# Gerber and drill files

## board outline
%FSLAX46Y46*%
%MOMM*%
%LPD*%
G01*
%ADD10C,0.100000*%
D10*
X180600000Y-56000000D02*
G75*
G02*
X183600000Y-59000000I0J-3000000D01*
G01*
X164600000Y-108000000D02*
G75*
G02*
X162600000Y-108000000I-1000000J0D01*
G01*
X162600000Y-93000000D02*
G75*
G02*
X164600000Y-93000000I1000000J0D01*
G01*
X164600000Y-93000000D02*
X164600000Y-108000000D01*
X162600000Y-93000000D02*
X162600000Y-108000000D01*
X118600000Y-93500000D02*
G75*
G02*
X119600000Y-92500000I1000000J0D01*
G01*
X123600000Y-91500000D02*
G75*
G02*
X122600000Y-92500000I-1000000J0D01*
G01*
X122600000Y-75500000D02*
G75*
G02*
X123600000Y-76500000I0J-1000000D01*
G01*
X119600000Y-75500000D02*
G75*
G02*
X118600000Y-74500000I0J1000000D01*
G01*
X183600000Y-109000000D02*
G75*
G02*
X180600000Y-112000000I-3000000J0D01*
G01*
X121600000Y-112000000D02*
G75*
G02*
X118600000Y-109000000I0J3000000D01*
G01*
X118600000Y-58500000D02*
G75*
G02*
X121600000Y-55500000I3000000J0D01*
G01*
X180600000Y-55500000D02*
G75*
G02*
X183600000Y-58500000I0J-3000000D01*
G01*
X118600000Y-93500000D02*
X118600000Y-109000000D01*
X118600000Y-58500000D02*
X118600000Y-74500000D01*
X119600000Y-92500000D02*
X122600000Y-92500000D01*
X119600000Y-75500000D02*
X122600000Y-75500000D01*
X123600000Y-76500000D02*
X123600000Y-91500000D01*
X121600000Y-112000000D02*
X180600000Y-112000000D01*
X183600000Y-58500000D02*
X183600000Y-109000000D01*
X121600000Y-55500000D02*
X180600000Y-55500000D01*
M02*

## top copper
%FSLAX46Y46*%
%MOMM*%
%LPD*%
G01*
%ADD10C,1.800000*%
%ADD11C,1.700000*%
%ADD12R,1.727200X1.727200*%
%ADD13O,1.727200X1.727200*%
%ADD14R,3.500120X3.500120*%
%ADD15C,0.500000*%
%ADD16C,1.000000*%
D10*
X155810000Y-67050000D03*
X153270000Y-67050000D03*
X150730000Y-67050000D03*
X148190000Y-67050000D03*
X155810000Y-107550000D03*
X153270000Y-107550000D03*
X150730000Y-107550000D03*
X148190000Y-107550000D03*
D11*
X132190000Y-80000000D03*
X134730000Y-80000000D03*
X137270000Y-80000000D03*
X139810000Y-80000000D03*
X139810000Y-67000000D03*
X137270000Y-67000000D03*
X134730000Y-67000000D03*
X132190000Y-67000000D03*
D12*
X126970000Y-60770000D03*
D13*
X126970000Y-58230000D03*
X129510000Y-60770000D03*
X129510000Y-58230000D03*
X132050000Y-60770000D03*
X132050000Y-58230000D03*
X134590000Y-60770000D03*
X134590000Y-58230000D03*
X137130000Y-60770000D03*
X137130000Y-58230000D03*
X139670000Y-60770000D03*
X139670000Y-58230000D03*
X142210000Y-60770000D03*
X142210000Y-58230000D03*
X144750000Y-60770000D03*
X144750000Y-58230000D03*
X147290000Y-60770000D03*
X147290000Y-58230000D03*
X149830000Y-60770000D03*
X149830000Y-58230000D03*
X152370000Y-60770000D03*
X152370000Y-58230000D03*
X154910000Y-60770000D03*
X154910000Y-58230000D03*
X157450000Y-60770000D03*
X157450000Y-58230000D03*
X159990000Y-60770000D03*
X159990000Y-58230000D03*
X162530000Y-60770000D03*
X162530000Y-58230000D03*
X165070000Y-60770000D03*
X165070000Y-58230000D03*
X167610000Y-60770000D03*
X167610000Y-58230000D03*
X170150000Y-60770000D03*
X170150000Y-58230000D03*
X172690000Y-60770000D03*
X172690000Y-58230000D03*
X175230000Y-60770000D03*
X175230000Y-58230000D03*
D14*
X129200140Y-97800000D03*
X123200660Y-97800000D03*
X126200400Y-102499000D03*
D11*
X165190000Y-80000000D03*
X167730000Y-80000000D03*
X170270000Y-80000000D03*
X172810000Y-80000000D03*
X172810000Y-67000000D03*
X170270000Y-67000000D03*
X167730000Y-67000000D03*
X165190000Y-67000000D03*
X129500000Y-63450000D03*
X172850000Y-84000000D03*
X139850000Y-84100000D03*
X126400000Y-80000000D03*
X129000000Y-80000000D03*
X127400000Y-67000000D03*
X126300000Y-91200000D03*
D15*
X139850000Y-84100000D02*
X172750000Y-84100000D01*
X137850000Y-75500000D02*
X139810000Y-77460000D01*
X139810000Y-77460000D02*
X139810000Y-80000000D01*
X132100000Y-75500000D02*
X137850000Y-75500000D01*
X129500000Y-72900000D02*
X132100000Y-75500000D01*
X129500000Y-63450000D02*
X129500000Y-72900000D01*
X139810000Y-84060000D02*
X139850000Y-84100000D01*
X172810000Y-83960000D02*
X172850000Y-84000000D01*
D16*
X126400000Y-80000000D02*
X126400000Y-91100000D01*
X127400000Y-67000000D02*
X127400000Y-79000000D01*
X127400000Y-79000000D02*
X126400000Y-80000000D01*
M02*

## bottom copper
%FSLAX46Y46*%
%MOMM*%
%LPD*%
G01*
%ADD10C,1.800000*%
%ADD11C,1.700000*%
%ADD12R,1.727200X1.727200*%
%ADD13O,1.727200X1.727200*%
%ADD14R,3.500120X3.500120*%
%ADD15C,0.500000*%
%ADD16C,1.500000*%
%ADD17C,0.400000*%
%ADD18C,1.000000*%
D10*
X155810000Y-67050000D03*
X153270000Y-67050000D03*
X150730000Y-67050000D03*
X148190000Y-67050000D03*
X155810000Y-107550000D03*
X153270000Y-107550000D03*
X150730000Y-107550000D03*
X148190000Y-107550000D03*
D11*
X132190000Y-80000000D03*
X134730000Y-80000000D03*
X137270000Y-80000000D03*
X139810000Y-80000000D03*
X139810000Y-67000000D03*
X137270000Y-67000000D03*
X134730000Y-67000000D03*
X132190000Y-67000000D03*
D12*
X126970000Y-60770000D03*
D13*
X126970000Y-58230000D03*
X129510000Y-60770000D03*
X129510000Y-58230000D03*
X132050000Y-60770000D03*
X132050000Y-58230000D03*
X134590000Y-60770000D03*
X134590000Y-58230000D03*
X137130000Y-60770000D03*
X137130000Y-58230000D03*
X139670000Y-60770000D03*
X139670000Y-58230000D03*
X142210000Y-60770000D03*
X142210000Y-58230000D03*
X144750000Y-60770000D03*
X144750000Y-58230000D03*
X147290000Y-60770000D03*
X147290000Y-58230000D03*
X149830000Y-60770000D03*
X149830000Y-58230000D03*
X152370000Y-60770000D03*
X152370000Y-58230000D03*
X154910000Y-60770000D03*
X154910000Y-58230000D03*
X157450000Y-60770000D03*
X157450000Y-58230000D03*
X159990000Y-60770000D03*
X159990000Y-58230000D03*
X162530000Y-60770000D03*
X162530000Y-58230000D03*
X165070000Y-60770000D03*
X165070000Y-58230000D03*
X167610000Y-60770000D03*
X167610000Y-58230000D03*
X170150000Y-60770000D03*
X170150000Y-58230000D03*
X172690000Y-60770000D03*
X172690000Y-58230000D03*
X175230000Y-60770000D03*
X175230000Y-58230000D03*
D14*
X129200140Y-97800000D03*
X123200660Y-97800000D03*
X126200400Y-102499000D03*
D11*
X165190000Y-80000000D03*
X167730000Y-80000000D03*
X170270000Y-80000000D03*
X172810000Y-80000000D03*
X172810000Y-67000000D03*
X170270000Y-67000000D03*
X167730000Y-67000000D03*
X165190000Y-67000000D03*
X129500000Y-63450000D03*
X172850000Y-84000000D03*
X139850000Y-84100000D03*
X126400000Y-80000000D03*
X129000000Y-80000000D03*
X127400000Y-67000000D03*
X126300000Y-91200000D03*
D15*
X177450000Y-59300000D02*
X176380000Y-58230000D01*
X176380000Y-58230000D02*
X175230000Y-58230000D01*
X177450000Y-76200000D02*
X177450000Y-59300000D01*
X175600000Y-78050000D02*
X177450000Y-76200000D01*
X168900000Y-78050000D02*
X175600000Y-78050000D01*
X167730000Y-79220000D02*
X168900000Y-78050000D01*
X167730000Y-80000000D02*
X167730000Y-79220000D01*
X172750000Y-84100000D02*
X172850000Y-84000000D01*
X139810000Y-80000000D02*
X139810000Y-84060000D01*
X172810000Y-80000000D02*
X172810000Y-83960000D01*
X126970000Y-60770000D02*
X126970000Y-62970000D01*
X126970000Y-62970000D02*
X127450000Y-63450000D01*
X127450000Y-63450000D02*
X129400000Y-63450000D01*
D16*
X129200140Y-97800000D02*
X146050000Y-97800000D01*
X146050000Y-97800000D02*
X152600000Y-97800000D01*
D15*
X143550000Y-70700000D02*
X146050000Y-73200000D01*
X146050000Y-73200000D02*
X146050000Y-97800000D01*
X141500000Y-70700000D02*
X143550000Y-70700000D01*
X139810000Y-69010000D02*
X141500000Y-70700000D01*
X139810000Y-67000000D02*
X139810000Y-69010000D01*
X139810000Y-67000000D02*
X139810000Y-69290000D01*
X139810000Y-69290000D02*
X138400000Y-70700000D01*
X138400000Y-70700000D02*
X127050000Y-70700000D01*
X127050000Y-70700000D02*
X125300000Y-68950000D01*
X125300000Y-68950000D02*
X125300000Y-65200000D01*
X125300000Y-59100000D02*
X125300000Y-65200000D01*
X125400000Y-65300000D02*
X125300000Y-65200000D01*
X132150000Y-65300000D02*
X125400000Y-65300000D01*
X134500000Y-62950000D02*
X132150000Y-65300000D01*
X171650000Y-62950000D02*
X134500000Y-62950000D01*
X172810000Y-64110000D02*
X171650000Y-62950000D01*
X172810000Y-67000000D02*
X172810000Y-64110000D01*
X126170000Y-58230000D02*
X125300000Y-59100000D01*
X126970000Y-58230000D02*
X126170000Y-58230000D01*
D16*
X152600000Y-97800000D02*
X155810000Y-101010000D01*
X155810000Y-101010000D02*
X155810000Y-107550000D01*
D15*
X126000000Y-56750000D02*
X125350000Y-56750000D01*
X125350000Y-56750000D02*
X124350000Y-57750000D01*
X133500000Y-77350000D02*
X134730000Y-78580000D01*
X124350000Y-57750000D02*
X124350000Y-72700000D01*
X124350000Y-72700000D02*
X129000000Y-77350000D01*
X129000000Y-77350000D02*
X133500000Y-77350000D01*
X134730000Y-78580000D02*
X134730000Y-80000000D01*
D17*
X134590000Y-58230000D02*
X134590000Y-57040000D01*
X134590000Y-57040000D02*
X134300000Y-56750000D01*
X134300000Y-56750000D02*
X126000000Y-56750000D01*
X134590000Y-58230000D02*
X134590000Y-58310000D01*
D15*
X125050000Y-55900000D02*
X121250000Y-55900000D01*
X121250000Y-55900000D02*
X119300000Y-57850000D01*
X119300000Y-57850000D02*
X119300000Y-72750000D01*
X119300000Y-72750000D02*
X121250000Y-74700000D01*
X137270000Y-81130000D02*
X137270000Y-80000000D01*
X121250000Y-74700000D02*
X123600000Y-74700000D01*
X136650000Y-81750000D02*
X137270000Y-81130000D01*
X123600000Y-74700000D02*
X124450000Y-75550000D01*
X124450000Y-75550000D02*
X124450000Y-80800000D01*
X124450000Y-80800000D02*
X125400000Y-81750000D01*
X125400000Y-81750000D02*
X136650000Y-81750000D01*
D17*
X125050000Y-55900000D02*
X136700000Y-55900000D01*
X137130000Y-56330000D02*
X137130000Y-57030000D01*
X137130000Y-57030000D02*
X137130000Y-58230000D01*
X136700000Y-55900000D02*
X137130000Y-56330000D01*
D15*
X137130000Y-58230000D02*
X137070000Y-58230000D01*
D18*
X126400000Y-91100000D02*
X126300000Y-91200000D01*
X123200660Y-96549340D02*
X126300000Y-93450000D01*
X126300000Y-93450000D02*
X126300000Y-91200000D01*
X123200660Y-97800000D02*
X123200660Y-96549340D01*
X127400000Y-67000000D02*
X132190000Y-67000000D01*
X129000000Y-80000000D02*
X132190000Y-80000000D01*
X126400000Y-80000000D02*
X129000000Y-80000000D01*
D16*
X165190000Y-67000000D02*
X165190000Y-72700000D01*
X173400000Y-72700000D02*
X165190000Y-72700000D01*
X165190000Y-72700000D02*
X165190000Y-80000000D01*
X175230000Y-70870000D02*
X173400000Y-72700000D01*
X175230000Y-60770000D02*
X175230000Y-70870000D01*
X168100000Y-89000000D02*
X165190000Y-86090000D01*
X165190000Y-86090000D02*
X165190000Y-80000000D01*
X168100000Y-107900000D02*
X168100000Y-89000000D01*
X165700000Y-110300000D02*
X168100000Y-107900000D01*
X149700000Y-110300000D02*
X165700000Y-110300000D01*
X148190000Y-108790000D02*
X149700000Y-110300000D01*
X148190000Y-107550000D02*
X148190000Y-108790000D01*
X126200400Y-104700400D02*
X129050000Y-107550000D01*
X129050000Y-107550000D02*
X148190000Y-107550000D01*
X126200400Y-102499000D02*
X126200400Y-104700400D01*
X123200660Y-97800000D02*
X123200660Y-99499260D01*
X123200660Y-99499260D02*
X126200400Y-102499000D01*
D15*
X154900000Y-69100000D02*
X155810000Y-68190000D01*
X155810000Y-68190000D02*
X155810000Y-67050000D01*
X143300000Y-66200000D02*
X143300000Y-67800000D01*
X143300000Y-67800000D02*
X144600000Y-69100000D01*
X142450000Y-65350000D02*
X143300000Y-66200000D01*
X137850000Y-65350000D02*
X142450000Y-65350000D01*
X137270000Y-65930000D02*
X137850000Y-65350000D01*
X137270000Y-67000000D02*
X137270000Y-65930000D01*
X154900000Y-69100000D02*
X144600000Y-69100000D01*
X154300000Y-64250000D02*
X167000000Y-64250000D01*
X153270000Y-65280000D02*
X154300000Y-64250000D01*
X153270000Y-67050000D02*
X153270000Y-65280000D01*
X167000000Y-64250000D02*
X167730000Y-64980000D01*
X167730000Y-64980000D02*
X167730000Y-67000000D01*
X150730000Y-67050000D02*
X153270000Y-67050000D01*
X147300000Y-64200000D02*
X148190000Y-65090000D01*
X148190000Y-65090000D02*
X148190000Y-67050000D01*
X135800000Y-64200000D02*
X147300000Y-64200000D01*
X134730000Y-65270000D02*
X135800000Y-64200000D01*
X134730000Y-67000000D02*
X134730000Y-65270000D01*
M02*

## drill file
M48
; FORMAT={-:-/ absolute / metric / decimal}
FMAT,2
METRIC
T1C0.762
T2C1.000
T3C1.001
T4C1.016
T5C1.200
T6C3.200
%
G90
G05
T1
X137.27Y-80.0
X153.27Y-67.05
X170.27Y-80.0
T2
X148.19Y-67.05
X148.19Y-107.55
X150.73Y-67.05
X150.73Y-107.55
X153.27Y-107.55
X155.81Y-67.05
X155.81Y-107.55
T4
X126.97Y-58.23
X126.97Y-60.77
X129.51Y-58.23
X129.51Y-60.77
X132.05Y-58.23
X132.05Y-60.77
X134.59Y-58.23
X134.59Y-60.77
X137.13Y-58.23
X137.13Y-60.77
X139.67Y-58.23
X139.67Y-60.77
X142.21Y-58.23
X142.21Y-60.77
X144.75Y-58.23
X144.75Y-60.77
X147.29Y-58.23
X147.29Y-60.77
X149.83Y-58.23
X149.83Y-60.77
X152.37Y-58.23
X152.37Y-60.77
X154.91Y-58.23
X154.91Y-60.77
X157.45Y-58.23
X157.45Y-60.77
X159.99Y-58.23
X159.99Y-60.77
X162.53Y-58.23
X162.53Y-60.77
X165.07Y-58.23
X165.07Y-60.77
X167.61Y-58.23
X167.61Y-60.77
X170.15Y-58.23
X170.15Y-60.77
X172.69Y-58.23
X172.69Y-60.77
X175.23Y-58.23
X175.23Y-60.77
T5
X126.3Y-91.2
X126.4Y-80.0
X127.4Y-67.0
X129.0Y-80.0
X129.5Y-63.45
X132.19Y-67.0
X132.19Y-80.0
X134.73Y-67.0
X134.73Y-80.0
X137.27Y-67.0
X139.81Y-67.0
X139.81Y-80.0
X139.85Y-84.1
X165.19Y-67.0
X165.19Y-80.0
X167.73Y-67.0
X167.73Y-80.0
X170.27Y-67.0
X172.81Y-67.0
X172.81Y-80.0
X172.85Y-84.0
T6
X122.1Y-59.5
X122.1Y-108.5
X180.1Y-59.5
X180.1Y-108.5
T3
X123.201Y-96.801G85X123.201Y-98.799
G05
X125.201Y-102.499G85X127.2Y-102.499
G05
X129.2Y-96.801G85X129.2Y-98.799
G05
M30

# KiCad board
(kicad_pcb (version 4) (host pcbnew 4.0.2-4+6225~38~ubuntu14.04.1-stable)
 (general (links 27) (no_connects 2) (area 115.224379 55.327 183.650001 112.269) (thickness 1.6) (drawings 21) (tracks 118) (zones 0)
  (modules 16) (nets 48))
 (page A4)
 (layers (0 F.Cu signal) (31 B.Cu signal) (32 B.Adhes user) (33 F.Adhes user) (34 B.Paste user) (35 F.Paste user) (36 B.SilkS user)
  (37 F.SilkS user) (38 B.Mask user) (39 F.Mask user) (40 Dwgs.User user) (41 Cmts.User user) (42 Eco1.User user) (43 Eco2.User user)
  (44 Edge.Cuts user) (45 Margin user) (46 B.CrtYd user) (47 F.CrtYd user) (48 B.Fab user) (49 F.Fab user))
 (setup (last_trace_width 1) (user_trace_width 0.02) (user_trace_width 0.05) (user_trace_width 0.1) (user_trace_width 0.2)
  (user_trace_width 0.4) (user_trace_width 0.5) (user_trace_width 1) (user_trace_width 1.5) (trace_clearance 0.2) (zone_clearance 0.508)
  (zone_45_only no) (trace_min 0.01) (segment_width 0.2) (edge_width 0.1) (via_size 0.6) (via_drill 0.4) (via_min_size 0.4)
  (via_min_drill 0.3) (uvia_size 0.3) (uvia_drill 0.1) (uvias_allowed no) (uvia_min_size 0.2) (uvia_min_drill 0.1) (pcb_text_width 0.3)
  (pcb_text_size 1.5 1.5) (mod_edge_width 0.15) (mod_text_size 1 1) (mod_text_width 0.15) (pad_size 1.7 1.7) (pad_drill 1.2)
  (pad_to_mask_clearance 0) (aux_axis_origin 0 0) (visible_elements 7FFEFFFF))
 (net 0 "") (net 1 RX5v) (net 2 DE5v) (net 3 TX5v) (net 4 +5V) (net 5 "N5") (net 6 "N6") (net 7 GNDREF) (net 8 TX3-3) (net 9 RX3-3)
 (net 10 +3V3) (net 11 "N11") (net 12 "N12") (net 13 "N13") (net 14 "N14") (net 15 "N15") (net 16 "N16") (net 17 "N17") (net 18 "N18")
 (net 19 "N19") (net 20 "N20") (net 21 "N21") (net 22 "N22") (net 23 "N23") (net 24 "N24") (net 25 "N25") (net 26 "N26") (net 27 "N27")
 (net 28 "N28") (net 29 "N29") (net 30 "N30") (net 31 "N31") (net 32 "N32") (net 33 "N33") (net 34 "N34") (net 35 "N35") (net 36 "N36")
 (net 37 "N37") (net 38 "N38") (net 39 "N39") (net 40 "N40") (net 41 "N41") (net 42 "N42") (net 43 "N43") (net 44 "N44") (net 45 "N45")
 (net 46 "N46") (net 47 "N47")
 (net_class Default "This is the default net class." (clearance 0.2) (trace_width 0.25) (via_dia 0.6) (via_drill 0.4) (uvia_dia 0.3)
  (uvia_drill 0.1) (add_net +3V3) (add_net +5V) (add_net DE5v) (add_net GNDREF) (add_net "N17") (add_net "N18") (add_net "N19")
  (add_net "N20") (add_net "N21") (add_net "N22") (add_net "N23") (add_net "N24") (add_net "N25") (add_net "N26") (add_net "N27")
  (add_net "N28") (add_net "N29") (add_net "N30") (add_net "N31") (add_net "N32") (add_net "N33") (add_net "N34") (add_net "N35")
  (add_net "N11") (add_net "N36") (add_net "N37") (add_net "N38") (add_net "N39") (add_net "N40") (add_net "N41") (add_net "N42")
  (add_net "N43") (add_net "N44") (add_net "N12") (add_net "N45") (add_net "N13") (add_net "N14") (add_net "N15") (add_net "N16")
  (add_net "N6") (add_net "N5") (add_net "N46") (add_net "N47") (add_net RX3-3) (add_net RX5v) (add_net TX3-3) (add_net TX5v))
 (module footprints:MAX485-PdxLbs (layer F.Cu) (at 152 87.3 180)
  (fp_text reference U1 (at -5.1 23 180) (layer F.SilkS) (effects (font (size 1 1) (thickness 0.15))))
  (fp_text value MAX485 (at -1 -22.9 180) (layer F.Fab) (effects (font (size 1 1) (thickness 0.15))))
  (pad 1 thru_hole circle (at -3.81 20.25 180) (size 1.8 1.8) (drill 1) (layers *.Cu *.Mask F.SilkS) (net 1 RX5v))
  (pad 2 thru_hole circle (at -1.27 20.25 180) (size 1.8 1.8) (drill 0.762) (layers *.Cu *.Mask F.SilkS) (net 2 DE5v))
  (pad 3 thru_hole circle (at 1.27 20.25 180) (size 1.8 1.8) (drill 1) (layers *.Cu *.Mask F.SilkS) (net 2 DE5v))
  (pad 4 thru_hole circle (at 3.81 20.25 180) (size 1.8 1.8) (drill 1) (layers *.Cu *.Mask F.SilkS) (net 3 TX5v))
  (pad 8 thru_hole circle (at -3.81 -20.25 180) (size 1.8 1.8) (drill 1) (layers *.Cu *.Mask F.SilkS) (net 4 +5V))
  (pad 7 thru_hole circle (at -1.27 -20.25 180) (size 1.8 1.8) (drill 1) (layers *.Cu *.Mask F.SilkS) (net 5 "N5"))
  (pad 6 thru_hole circle (at 1.27 -20.25 180) (size 1.8 1.8) (drill 1) (layers *.Cu *.Mask F.SilkS) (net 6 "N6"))
  (pad 5 thru_hole circle (at 3.81 -20.25 180) (size 1.8 1.8) (drill 1) (layers *.Cu *.Mask F.SilkS) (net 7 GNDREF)))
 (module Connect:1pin (layer F.Cu) (at 180.1 59.5)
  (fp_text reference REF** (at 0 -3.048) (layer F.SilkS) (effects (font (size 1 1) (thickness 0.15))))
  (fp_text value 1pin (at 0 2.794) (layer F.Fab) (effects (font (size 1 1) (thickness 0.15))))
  (pad "" np_thru_hole circle (at 0 0) (size 3.2 3.2) (drill 3.2) (layers *.Cu *.Mask F.SilkS)))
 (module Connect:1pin (layer F.Cu) (at 180.1 108.5)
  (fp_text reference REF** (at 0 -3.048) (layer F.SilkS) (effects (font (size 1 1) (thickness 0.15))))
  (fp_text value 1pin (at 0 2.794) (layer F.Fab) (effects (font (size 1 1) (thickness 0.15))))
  (pad "" np_thru_hole circle (at 0 0) (size 3.2 3.2) (drill 3.2) (layers *.Cu *.Mask F.SilkS)))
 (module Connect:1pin (layer F.Cu) (at 122.1 108.5)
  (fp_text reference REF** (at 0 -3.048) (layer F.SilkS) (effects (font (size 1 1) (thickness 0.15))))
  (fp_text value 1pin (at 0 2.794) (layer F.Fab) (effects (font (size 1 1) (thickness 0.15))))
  (pad "" np_thru_hole circle (at 0 0) (size 3.2 3.2) (drill 3.2) (layers *.Cu *.Mask F.SilkS)))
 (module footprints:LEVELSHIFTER (layer F.Cu) (at 136 73.5 90)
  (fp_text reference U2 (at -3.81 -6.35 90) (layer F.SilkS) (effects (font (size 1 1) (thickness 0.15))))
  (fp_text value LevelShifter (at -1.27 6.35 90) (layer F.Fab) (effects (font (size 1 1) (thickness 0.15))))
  (pad 1 thru_hole circle (at -6.5 -3.81 90) (size 1.7 1.7) (drill 1.2) (layers *.Cu *.Mask F.SilkS) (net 7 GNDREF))
  (pad 2 thru_hole circle (at -6.5 -1.27 90) (size 1.7 1.7) (drill 1.2) (layers *.Cu *.Mask F.SilkS) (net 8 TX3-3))
  (pad 3 thru_hole circle (at -6.5 1.27 90) (size 1.7 1.7) (drill 0.762) (layers *.Cu *.Mask F.SilkS) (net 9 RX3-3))
  (pad 4 thru_hole circle (at -6.5 3.81 90) (size 1.7 1.7) (drill 1.2) (layers *.Cu *.Mask F.SilkS) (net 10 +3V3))
  (pad 5 thru_hole circle (at 6.5 3.81 90) (size 1.7 1.7) (drill 1.2) (layers *.Cu *.Mask F.SilkS) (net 4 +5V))
  (pad 6 thru_hole circle (at 6.5 1.27 90) (size 1.7 1.7) (drill 1.2) (layers *.Cu *.Mask F.SilkS) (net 1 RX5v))
  (pad 7 thru_hole circle (at 6.5 -1.27 90) (size 1.7 1.7) (drill 1.2) (layers *.Cu *.Mask F.SilkS) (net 3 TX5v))
  (pad 8 thru_hole circle (at 6.5 -3.81 90) (size 1.7 1.7) (drill 1.2) (layers *.Cu *.Mask F.SilkS) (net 7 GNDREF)))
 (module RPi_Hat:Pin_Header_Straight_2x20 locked (layer F.Cu) (at 151.1 59.5 90)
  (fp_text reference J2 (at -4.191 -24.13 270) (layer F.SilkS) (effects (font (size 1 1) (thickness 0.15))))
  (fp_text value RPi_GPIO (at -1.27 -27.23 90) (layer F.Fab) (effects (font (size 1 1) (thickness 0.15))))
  (pad 1 thru_hole rect (at -1.27 -24.13 90) (size 1.7272 1.7272) (drill 1.016) (layers *.Cu *.Mask F.SilkS) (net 10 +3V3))
  (pad 2 thru_hole oval (at 1.27 -24.13 90) (size 1.7272 1.7272) (drill 1.016) (layers *.Cu *.Mask F.SilkS) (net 4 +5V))
  (pad 3 thru_hole oval (at -1.27 -21.59 90) (size 1.7272 1.7272) (drill 1.016) (layers *.Cu *.Mask F.SilkS) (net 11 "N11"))
  (pad 4 thru_hole oval (at 1.27 -21.59 90) (size 1.7272 1.7272) (drill 1.016) (layers *.Cu *.Mask F.SilkS) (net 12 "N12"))
  (pad 5 thru_hole oval (at -1.27 -19.05 90) (size 1.7272 1.7272) (drill 1.016) (layers *.Cu *.Mask F.SilkS) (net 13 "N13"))
  (pad 6 thru_hole oval (at 1.27 -19.05 90) (size 1.7272 1.7272) (drill 1.016) (layers *.Cu *.Mask F.SilkS) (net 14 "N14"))
  (pad 7 thru_hole oval (at -1.27 -16.51 90) (size 1.7272 1.7272) (drill 1.016) (layers *.Cu *.Mask F.SilkS) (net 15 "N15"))
  (pad 8 thru_hole oval (at 1.27 -16.51 90) (size 1.7272 1.7272) (drill 1.016) (layers *.Cu *.Mask F.SilkS) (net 8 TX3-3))
  (pad 9 thru_hole oval (at -1.27 -13.97 90) (size 1.7272 1.7272) (drill 1.016) (layers *.Cu *.Mask F.SilkS) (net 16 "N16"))
  (pad 10 thru_hole oval (at 1.27 -13.97 90) (size 1.7272 1.7272) (drill 1.016) (layers *.Cu *.Mask F.SilkS) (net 9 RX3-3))
  (pad 11 thru_hole oval (at -1.27 -11.43 90) (size 1.7272 1.7272) (drill 1.016) (layers *.Cu *.Mask F.SilkS) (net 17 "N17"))
  (pad 12 thru_hole oval (at 1.27 -11.43 90) (size 1.7272 1.7272) (drill 1.016) (layers *.Cu *.Mask F.SilkS) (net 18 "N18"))
  (pad 13 thru_hole oval (at -1.27 -8.89 90) (size 1.7272 1.7272) (drill 1.016) (layers *.Cu *.Mask F.SilkS) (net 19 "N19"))
  (pad 14 thru_hole oval (at 1.27 -8.89 90) (size 1.7272 1.7272) (drill 1.016) (layers *.Cu *.Mask F.SilkS) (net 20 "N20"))
  (pad 15 thru_hole oval (at -1.27 -6.35 90) (size 1.7272 1.7272) (drill 1.016) (layers *.Cu *.Mask F.SilkS) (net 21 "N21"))
  (pad 16 thru_hole oval (at 1.27 -6.35 90) (size 1.7272 1.7272) (drill 1.016) (layers *.Cu *.Mask F.SilkS) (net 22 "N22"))
  (pad 17 thru_hole oval (at -1.27 -3.81 90) (size 1.7272 1.7272) (drill 1.016) (layers *.Cu *.Mask F.SilkS) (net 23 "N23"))
  (pad 18 thru_hole oval (at 1.27 -3.81 90) (size 1.7272 1.7272) (drill 1.016) (layers *.Cu *.Mask F.SilkS) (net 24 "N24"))
  (pad 19 thru_hole oval (at -1.27 -1.27 90) (size 1.7272 1.7272) (drill 1.016) (layers *.Cu *.Mask F.SilkS) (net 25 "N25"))
  (pad 20 thru_hole oval (at 1.27 -1.27 90) (size 1.7272 1.7272) (drill 1.016) (layers *.Cu *.Mask F.SilkS) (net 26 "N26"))
  (pad 21 thru_hole oval (at -1.27 1.27 90) (size 1.7272 1.7272) (drill 1.016) (layers *.Cu *.Mask F.SilkS) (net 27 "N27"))
  (pad 22 thru_hole oval (at 1.27 1.27 90) (size 1.7272 1.7272) (drill 1.016) (layers *.Cu *.Mask F.SilkS) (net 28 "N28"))
  (pad 23 thru_hole oval (at -1.27 3.81 90) (size 1.7272 1.7272) (drill 1.016) (layers *.Cu *.Mask F.SilkS) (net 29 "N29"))
  (pad 24 thru_hole oval (at 1.27 3.81 90) (size 1.7272 1.7272) (drill 1.016) (layers *.Cu *.Mask F.SilkS) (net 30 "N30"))
  (pad 25 thru_hole oval (at -1.27 6.35 90) (size 1.7272 1.7272) (drill 1.016) (layers *.Cu *.Mask F.SilkS) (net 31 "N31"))
  (pad 26 thru_hole oval (at 1.27 6.35 90) (size 1.7272 1.7272) (drill 1.016) (layers *.Cu *.Mask F.SilkS) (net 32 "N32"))
  (pad 27 thru_hole oval (at -1.27 8.89 90) (size 1.7272 1.7272) (drill 1.016) (layers *.Cu *.Mask F.SilkS) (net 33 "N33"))
  (pad 28 thru_hole oval (at 1.27 8.89 90) (size 1.7272 1.7272) (drill 1.016) (layers *.Cu *.Mask F.SilkS) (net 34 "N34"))
  (pad 29 thru_hole oval (at -1.27 11.43 90) (size 1.7272 1.7272) (drill 1.016) (layers *.Cu *.Mask F.SilkS) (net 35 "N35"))
  (pad 30 thru_hole oval (at 1.27 11.43 90) (size 1.7272 1.7272) (drill 1.016) (layers *.Cu *.Mask F.SilkS) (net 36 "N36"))
  (pad 31 thru_hole oval (at -1.27 13.97 90) (size 1.7272 1.7272) (drill 1.016) (layers *.Cu *.Mask F.SilkS) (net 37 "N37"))
  (pad 32 thru_hole oval (at 1.27 13.97 90) (size 1.7272 1.7272) (drill 1.016) (layers *.Cu *.Mask F.SilkS) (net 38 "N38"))
  (pad 33 thru_hole oval (at -1.27 16.51 90) (size 1.7272 1.7272) (drill 1.016) (layers *.Cu *.Mask F.SilkS) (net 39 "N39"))
  (pad 34 thru_hole oval (at 1.27 16.51 90) (size 1.7272 1.7272) (drill 1.016) (layers *.Cu *.Mask F.SilkS) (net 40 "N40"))
  (pad 35 thru_hole oval (at -1.27 19.05 90) (size 1.7272 1.7272) (drill 1.016) (layers *.Cu *.Mask F.SilkS) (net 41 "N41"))
  (pad 36 thru_hole oval (at 1.27 19.05 90) (size 1.7272 1.7272) (drill 1.016) (layers *.Cu *.Mask F.SilkS) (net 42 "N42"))
  (pad 37 thru_hole oval (at -1.27 21.59 90) (size 1.7272 1.7272) (drill 1.016) (layers *.Cu *.Mask F.SilkS) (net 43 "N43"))
  (pad 38 thru_hole oval (at 1.27 21.59 90) (size 1.7272 1.7272) (drill 1.016) (layers *.Cu *.Mask F.SilkS) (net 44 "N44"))
  (pad 39 thru_hole oval (at -1.27 24.13 90) (size 1.7272 1.7272) (drill 1.016) (layers *.Cu *.Mask F.SilkS) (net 7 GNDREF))
  (pad 40 thru_hole oval (at 1.27 24.13 90) (size 1.7272 1.7272) (drill 1.016) (layers *.Cu *.Mask F.SilkS) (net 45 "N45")))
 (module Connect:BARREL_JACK (layer F.Cu) (at 123 97.8)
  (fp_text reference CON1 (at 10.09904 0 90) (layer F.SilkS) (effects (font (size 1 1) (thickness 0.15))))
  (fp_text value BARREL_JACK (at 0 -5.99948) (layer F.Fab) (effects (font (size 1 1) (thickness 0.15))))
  (pad 1 thru_hole rect (at 6.20014 0) (size 3.50012 3.50012) (drill oval 1.00076 2.99974) (layers *.Cu *.Mask F.SilkS) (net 4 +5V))
  (pad 2 thru_hole rect (at 0.20066 0) (size 3.50012 3.50012) (drill oval 1.00076 2.99974) (layers *.Cu *.Mask F.SilkS) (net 7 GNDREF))
  (pad 3 thru_hole rect (at 3.2004 4.699) (size 3.50012 3.50012) (drill oval 2.99974 1.00076) (layers *.Cu *.Mask F.SilkS) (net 7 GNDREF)))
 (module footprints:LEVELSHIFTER (layer F.Cu) (at 169 73.5 90)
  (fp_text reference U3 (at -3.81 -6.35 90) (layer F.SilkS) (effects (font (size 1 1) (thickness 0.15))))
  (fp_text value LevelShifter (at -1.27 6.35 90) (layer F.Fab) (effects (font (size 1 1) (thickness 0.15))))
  (pad 1 thru_hole circle (at -6.5 -3.81 90) (size 1.7 1.7) (drill 1.2) (layers *.Cu *.Mask F.SilkS) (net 7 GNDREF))
  (pad 2 thru_hole circle (at -6.5 -1.27 90) (size 1.7 1.7) (drill 1.2) (layers *.Cu *.Mask F.SilkS) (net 45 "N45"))
  (pad 3 thru_hole circle (at -6.5 1.27 90) (size 1.7 1.7) (drill 0.762) (layers *.Cu *.Mask F.SilkS) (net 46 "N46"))
  (pad 4 thru_hole circle (at -6.5 3.81 90) (size 1.7 1.7) (drill 1.2) (layers *.Cu *.Mask F.SilkS) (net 10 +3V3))
  (pad 5 thru_hole circle (at 6.5 3.81 90) (size 1.7 1.7) (drill 1.2) (layers *.Cu *.Mask F.SilkS) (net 4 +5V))
  (pad 6 thru_hole circle (at 6.5 1.27 90) (size 1.7 1.7) (drill 1.2) (layers *.Cu *.Mask F.SilkS) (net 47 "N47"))
  (pad 7 thru_hole circle (at 6.5 -1.27 90) (size 1.7 1.7) (drill 1.2) (layers *.Cu *.Mask F.SilkS) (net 2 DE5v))
  (pad 8 thru_hole circle (at 6.5 -3.81 90) (size 1.7 1.7) (drill 1.2) (layers *.Cu *.Mask F.SilkS) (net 7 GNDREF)))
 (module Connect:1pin (layer F.Cu) (at 122.1 59.5)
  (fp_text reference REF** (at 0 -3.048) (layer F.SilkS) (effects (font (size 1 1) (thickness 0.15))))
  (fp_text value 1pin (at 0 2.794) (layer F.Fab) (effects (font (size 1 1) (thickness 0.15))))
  (pad "" np_thru_hole circle (at 0 0) (size 3.2 3.2) (drill 3.2) (layers *.Cu *.Mask F.SilkS)))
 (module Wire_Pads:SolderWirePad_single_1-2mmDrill (layer F.Cu) (at 129.5 63.45)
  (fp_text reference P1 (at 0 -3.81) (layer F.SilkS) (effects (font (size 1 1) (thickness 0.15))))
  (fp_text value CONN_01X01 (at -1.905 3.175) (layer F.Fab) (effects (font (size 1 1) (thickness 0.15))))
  (pad 1 thru_hole circle (at 0 0) (size 1.7 1.7) (drill 1.2) (layers *.Cu *.Mask F.SilkS) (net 10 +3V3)))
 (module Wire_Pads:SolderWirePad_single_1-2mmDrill (layer F.Cu) (at 172.85 84)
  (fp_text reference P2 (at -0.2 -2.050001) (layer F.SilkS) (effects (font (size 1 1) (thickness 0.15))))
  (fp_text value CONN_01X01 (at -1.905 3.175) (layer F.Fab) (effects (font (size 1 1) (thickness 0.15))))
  (pad 1 thru_hole circle (at 0 0) (size 1.7 1.7) (drill 1.2) (layers *.Cu *.Mask F.SilkS) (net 10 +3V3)))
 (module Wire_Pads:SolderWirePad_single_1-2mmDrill (layer F.Cu) (at 139.85 84.1)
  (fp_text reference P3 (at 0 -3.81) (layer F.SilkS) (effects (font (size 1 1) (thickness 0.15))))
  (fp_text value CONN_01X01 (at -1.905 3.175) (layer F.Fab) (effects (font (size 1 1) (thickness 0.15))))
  (pad 1 thru_hole circle (at 0 0) (size 1.7 1.7) (drill 1.2) (layers *.Cu *.Mask F.SilkS) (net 10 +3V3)))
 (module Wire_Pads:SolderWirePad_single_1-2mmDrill (layer F.Cu) (at 126.4 80)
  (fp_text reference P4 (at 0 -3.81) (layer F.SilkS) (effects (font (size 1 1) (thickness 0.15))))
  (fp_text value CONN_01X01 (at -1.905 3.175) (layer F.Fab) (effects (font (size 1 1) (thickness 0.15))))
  (pad 1 thru_hole circle (at 0 0) (size 1.7 1.7) (drill 1.2) (layers *.Cu *.Mask F.SilkS) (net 7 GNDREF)))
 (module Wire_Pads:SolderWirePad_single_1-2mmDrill (layer F.Cu) (at 129 80)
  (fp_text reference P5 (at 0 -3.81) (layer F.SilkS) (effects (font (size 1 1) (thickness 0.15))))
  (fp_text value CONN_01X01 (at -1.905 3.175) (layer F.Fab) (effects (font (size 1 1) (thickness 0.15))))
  (pad 1 thru_hole circle (at 0 0) (size 1.7 1.7) (drill 1.2) (layers *.Cu *.Mask F.SilkS) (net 7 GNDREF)))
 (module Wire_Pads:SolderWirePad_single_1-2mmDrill (layer F.Cu) (at 127.4 67)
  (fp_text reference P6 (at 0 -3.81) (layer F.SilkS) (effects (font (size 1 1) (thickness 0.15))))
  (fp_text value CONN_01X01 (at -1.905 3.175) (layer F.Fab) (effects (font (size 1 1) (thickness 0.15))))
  (pad 1 thru_hole circle (at 0 0) (size 1.7 1.7) (drill 1.2) (layers *.Cu *.Mask F.SilkS) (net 7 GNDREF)))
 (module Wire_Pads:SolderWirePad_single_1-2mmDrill (layer F.Cu) (at 126.3 91.2)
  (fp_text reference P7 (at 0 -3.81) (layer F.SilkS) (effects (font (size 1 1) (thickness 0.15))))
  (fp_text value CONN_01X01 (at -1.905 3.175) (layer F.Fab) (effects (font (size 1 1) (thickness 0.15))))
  (pad 1 thru_hole circle (at 0 0) (size 1.7 1.7) (drill 1.2) (layers *.Cu *.Mask F.SilkS) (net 7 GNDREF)))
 (gr_arc (start 180.6 59) (end 180.6 56) (angle 90) (layer Edge.Cuts) (width 0.1))
 (gr_arc (start 163.6 108) (end 162.6 108) (angle -180) (layer Edge.Cuts) (width 0.1))
 (gr_arc (start 163.6 93) (end 162.6 93) (angle 180) (layer Edge.Cuts) (width 0.1))
 (gr_line (start 164.6 93) (end 164.6 108) (angle 90) (layer Edge.Cuts) (width 0.1))
 (gr_line (start 162.6 93) (end 162.6 108) (angle 90) (layer Edge.Cuts) (width 0.1))
 (gr_arc (start 119.6 93.5) (end 118.6 93.5) (angle 90) (layer Edge.Cuts) (width 0.1))
 (gr_arc (start 122.6 91.5) (end 123.6 91.5) (angle 90) (layer Edge.Cuts) (width 0.1))
 (gr_arc (start 122.6 76.5) (end 122.6 75.5) (angle 90) (layer Edge.Cuts) (width 0.1))
 (gr_arc (start 119.6 74.5) (end 119.6 75.5) (angle 90) (layer Edge.Cuts) (width 0.1))
 (gr_arc (start 180.6 109) (end 183.6 109) (angle 90) (layer Edge.Cuts) (width 0.1))
 (gr_arc (start 121.6 109) (end 121.6 112) (angle 90) (layer Edge.Cuts) (width 0.1))
 (gr_arc (start 121.6 58.5) (end 118.6 58.5) (angle 90) (layer Edge.Cuts) (width 0.1))
 (gr_arc (start 180.6 58.5) (end 180.6 55.5) (angle 90) (layer Edge.Cuts) (width 0.1))
 (gr_line (start 118.6 93.5) (end 118.6 109) (layer Edge.Cuts) (width 0.1))
 (gr_line (start 118.6 58.5) (end 118.6 74.5) (layer Edge.Cuts) (width 0.1))
 (gr_line (start 119.6 92.5) (end 122.6 92.5) (layer Edge.Cuts) (width 0.1))
 (gr_line (start 119.6 75.5) (end 122.6 75.5) (layer Edge.Cuts) (width 0.1))
 (gr_line (start 123.6 76.5) (end 123.6 91.5) (layer Edge.Cuts) (width 0.1))
 (gr_line (start 121.6 112) (end 180.6 112) (angle 90) (layer Edge.Cuts) (width 0.1))
 (gr_line (start 183.6 58.5) (end 183.6 109) (angle 90) (layer Edge.Cuts) (width 0.1))
 (gr_line (start 121.6 55.5) (end 180.6 55.5) (angle 90) (layer Edge.Cuts) (width 0.1))
 (segment (start 177.45 59.3) (end 176.38 58.23) (width 0.5) (layer B.Cu) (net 45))
 (segment (start 176.38 58.23) (end 175.23 58.23) (width 0.5) (layer B.Cu) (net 45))
 (segment (start 177.45 76.2) (end 177.45 59.3) (width 0.5) (layer B.Cu) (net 45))
 (segment (start 175.6 78.05) (end 177.45 76.2) (width 0.5) (layer B.Cu) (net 45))
 (segment (start 168.9 78.05) (end 175.6 78.05) (width 0.5) (layer B.Cu) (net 45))
 (segment (start 167.73 79.22) (end 168.9 78.05) (width 0.5) (layer B.Cu) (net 45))
 (segment (start 167.73 80) (end 167.73 79.22) (width 0.5) (layer B.Cu) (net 45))
 (segment (start 139.85 84.1) (end 172.75 84.1) (width 0.5) (layer F.Cu) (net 10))
 (segment (start 172.75 84.1) (end 172.85 84) (width 0.5) (layer B.Cu) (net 10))
 (segment (start 137.85 75.5) (end 139.81 77.46) (width 0.5) (layer F.Cu) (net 10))
 (segment (start 139.81 77.46) (end 139.81 80) (width 0.5) (layer F.Cu) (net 10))
 (segment (start 132.1 75.5) (end 137.85 75.5) (width 0.5) (layer F.Cu) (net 10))
 (segment (start 129.5 72.9) (end 132.1 75.5) (width 0.5) (layer F.Cu) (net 10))
 (segment (start 129.5 63.45) (end 129.5 72.9) (width 0.5) (layer F.Cu) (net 10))
 (segment (start 139.81 80) (end 139.81 84.06) (width 0.5) (layer B.Cu) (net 10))
 (segment (start 139.81 84.06) (end 139.85 84.1) (width 0.5) (layer F.Cu) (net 10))
 (segment (start 172.81 80) (end 172.81 83.96) (width 0.5) (layer B.Cu) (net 10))
 (segment (start 172.81 83.96) (end 172.85 84) (width 0.5) (layer F.Cu) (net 10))
 (segment (start 126.97 60.77) (end 126.97 62.97) (width 0.5) (layer B.Cu) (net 10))
 (segment (start 126.97 62.97) (end 127.45 63.45) (width 0.5) (layer B.Cu) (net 10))
 (segment (start 127.45 63.45) (end 129.4 63.45) (width 0.5) (layer B.Cu) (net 10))
 (segment (start 129.20014 97.8) (end 146.05 97.8) (width 1.5) (layer B.Cu) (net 4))
 (segment (start 146.05 97.8) (end 152.6 97.8) (width 1.5) (layer B.Cu) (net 4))
 (segment (start 143.55 70.7) (end 146.05 73.2) (width 0.5) (layer B.Cu) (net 4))
 (segment (start 146.05 73.2) (end 146.05 97.8) (width 0.5) (layer B.Cu) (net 4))
 (segment (start 141.5 70.7) (end 143.55 70.7) (width 0.5) (layer B.Cu) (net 4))
 (segment (start 139.81 69.01) (end 141.5 70.7) (width 0.5) (layer B.Cu) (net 4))
 (segment (start 139.81 67) (end 139.81 69.01) (width 0.5) (layer B.Cu) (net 4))
 (segment (start 139.81 67) (end 139.81 69.29) (width 0.5) (layer B.Cu) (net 4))
 (segment (start 139.81 69.29) (end 138.4 70.7) (width 0.5) (layer B.Cu) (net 4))
 (segment (start 138.4 70.7) (end 127.05 70.7) (width 0.5) (layer B.Cu) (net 4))
 (segment (start 127.05 70.7) (end 125.3 68.95) (width 0.5) (layer B.Cu) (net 4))
 (segment (start 125.3 68.95) (end 125.3 65.2) (width 0.5) (layer B.Cu) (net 4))
 (segment (start 125.3 59.1) (end 125.3 65.2) (width 0.5) (layer B.Cu) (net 4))
 (segment (start 125.4 65.3) (end 125.3 65.2) (width 0.5) (layer B.Cu) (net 4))
 (segment (start 132.15 65.3) (end 125.4 65.3) (width 0.5) (layer B.Cu) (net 4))
 (segment (start 134.5 62.95) (end 132.15 65.3) (width 0.5) (layer B.Cu) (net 4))
 (segment (start 171.65 62.95) (end 134.5 62.95) (width 0.5) (layer B.Cu) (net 4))
 (segment (start 172.81 64.11) (end 171.65 62.95) (width 0.5) (layer B.Cu) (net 4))
 (segment (start 172.81 67) (end 172.81 64.11) (width 0.5) (layer B.Cu) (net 4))
 (segment (start 126.17 58.23) (end 125.3 59.1) (width 0.5) (layer B.Cu) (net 4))
 (segment (start 126.97 58.23) (end 126.17 58.23) (width 0.5) (layer B.Cu) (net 4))
 (segment (start 152.6 97.8) (end 155.81 101.01) (width 1.5) (layer B.Cu) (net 4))
 (segment (start 155.81 101.01) (end 155.81 107.55) (width 1.5) (layer B.Cu) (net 4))
 (segment (start 126 56.75) (end 125.35 56.75) (width 0.5) (layer B.Cu) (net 8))
 (segment (start 125.35 56.75) (end 124.35 57.75) (width 0.5) (layer B.Cu) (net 8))
 (segment (start 133.5 77.35) (end 134.73 78.58) (width 0.5) (layer B.Cu) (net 8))
 (segment (start 124.35 57.75) (end 124.35 72.7) (width 0.5) (layer B.Cu) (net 8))
 (segment (start 124.35 72.7) (end 129 77.35) (width 0.5) (layer B.Cu) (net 8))
 (segment (start 129 77.35) (end 133.5 77.35) (width 0.5) (layer B.Cu) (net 8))
 (segment (start 134.73 78.58) (end 134.73 80) (width 0.5) (layer B.Cu) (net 8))
 (segment (start 134.59 58.23) (end 134.59 57.04) (width 0.4) (layer B.Cu) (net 8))
 (segment (start 134.59 57.04) (end 134.3 56.75) (width 0.4) (layer B.Cu) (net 8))
 (segment (start 134.3 56.75) (end 126 56.75) (width 0.4) (layer B.Cu) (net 8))
 (segment (start 134.59 58.23) (end 134.59 58.31) (width 0.4) (layer B.Cu) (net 8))
 (segment (start 125.05 55.9) (end 121.25 55.9) (width 0.5) (layer B.Cu) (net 9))
 (segment (start 121.25 55.9) (end 119.3 57.85) (width 0.5) (layer B.Cu) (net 9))
 (segment (start 119.3 57.85) (end 119.3 72.75) (width 0.5) (layer B.Cu) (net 9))
 (segment (start 119.3 72.75) (end 121.25 74.7) (width 0.5) (layer B.Cu) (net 9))
 (segment (start 137.27 81.13) (end 137.27 80) (width 0.5) (layer B.Cu) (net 9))
 (segment (start 121.25 74.7) (end 123.6 74.7) (width 0.5) (layer B.Cu) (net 9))
 (segment (start 136.65 81.75) (end 137.27 81.13) (width 0.5) (layer B.Cu) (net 9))
 (segment (start 123.6 74.7) (end 124.45 75.55) (width 0.5) (layer B.Cu) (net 9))
 (segment (start 124.45 75.55) (end 124.45 80.8) (width 0.5) (layer B.Cu) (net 9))
 (segment (start 124.45 80.8) (end 125.4 81.75) (width 0.5) (layer B.Cu) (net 9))
 (segment (start 125.4 81.75) (end 136.65 81.75) (width 0.5) (layer B.Cu) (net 9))
 (segment (start 125.05 55.9) (end 136.7 55.9) (width 0.4) (layer B.Cu) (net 9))
 (segment (start 137.13 56.33) (end 137.13 57.03) (width 0.4) (layer B.Cu) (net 9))
 (segment (start 137.13 57.03) (end 137.13 58.23) (width 0.4) (layer B.Cu) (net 9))
 (segment (start 136.7 55.9) (end 137.13 56.33) (width 0.4) (layer B.Cu) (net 9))
 (segment (start 137.13 58.23) (end 137.07 58.23) (width 0.5) (layer B.Cu) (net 9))
 (segment (start 126.4 80) (end 126.4 91.1) (width 1) (layer F.Cu) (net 7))
 (segment (start 126.4 91.1) (end 126.3 91.2) (width 1) (layer B.Cu) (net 7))
 (segment (start 123.20066 96.54934) (end 126.3 93.45) (width 1) (layer B.Cu) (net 7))
 (segment (start 126.3 93.45) (end 126.3 91.2) (width 1) (layer B.Cu) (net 7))
 (segment (start 123.20066 97.8) (end 123.20066 96.54934) (width 1) (layer B.Cu) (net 7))
 (segment (start 127.4 67) (end 127.4 79) (width 1) (layer F.Cu) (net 7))
 (segment (start 127.4 79) (end 126.4 80) (width 1) (layer F.Cu) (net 7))
 (segment (start 127.4 67) (end 132.19 67) (width 1) (layer B.Cu) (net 7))
 (segment (start 129 80) (end 132.19 80) (width 1) (layer B.Cu) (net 7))
 (segment (start 126.4 80) (end 129 80) (width 1) (layer B.Cu) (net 7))
 (segment (start 165.19 67) (end 165.19 72.7) (width 1.5) (layer B.Cu) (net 7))
 (segment (start 173.4 72.7) (end 165.19 72.7) (width 1.5) (layer B.Cu) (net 7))
 (segment (start 165.19 72.7) (end 165.19 80) (width 1.5) (layer B.Cu) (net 7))
 (segment (start 175.23 70.87) (end 173.4 72.7) (width 1.5) (layer B.Cu) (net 7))
 (segment (start 175.23 60.77) (end 175.23 70.87) (width 1.5) (layer B.Cu) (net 7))
 (segment (start 168.1 89) (end 165.19 86.09) (width 1.5) (layer B.Cu) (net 7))
 (segment (start 165.19 86.09) (end 165.19 80) (width 1.5) (layer B.Cu) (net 7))
 (segment (start 168.1 107.9) (end 168.1 89) (width 1.5) (layer B.Cu) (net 7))
 (segment (start 165.7 110.3) (end 168.1 107.9) (width 1.5) (layer B.Cu) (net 7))
 (segment (start 149.7 110.3) (end 165.7 110.3) (width 1.5) (layer B.Cu) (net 7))
 (segment (start 148.19 108.79) (end 149.7 110.3) (width 1.5) (layer B.Cu) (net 7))
 (segment (start 148.19 107.55) (end 148.19 108.79) (width 1.5) (layer B.Cu) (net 7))
 (segment (start 126.2004 104.7004) (end 129.05 107.55) (width 1.5) (layer B.Cu) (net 7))
 (segment (start 129.05 107.55) (end 148.19 107.55) (width 1.5) (layer B.Cu) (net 7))
 (segment (start 126.2004 102.499) (end 126.2004 104.7004) (width 1.5) (layer B.Cu) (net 7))
 (segment (start 123.20066 97.8) (end 123.20066 99.49926) (width 1.5) (layer B.Cu) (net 7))
 (segment (start 123.20066 99.49926) (end 126.2004 102.499) (width 1.5) (layer B.Cu) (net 7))
 (segment (start 154.9 69.1) (end 155.81 68.19) (width 0.5) (layer B.Cu) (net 1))
 (segment (start 155.81 68.19) (end 155.81 67.05) (width 0.5) (layer B.Cu) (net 1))
 (segment (start 143.3 66.2) (end 143.3 67.8) (width 0.5) (layer B.Cu) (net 1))
 (segment (start 143.3 67.8) (end 144.6 69.1) (width 0.5) (layer B.Cu) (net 1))
 (segment (start 142.45 65.35) (end 143.3 66.2) (width 0.5) (layer B.Cu) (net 1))
 (segment (start 137.85 65.35) (end 142.45 65.35) (width 0.5) (layer B.Cu) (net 1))
 (segment (start 137.27 65.93) (end 137.85 65.35) (width 0.5) (layer B.Cu) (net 1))
 (segment (start 137.27 67) (end 137.27 65.93) (width 0.5) (layer B.Cu) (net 1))
 (segment (start 154.9 69.1) (end 144.6 69.1) (width 0.5) (layer B.Cu) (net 1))
 (segment (start 154.3 64.25) (end 167 64.25) (width 0.5) (layer B.Cu) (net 2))
 (segment (start 153.27 65.28) (end 154.3 64.25) (width 0.5) (layer B.Cu) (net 2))
 (segment (start 153.27 67.05) (end 153.27 65.28) (width 0.5) (layer B.Cu) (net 2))
 (segment (start 167 64.25) (end 167.73 64.98) (width 0.5) (layer B.Cu) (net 2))
 (segment (start 167.73 64.98) (end 167.73 67) (width 0.5) (layer B.Cu) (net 2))
 (segment (start 150.73 67.05) (end 153.27 67.05) (width 0.5) (layer B.Cu) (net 2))
 (segment (start 147.3 64.2) (end 148.19 65.09) (width 0.5) (layer B.Cu) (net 3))
 (segment (start 148.19 65.09) (end 148.19 67.05) (width 0.5) (layer B.Cu) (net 3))
 (segment (start 135.8 64.2) (end 147.3 64.2) (width 0.5) (layer B.Cu) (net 3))
 (segment (start 134.73 65.27) (end 135.8 64.2) (width 0.5) (layer B.Cu) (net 3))
 (segment (start 134.73 67) (end 134.73 65.27) (width 0.5) (layer B.Cu) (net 3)))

